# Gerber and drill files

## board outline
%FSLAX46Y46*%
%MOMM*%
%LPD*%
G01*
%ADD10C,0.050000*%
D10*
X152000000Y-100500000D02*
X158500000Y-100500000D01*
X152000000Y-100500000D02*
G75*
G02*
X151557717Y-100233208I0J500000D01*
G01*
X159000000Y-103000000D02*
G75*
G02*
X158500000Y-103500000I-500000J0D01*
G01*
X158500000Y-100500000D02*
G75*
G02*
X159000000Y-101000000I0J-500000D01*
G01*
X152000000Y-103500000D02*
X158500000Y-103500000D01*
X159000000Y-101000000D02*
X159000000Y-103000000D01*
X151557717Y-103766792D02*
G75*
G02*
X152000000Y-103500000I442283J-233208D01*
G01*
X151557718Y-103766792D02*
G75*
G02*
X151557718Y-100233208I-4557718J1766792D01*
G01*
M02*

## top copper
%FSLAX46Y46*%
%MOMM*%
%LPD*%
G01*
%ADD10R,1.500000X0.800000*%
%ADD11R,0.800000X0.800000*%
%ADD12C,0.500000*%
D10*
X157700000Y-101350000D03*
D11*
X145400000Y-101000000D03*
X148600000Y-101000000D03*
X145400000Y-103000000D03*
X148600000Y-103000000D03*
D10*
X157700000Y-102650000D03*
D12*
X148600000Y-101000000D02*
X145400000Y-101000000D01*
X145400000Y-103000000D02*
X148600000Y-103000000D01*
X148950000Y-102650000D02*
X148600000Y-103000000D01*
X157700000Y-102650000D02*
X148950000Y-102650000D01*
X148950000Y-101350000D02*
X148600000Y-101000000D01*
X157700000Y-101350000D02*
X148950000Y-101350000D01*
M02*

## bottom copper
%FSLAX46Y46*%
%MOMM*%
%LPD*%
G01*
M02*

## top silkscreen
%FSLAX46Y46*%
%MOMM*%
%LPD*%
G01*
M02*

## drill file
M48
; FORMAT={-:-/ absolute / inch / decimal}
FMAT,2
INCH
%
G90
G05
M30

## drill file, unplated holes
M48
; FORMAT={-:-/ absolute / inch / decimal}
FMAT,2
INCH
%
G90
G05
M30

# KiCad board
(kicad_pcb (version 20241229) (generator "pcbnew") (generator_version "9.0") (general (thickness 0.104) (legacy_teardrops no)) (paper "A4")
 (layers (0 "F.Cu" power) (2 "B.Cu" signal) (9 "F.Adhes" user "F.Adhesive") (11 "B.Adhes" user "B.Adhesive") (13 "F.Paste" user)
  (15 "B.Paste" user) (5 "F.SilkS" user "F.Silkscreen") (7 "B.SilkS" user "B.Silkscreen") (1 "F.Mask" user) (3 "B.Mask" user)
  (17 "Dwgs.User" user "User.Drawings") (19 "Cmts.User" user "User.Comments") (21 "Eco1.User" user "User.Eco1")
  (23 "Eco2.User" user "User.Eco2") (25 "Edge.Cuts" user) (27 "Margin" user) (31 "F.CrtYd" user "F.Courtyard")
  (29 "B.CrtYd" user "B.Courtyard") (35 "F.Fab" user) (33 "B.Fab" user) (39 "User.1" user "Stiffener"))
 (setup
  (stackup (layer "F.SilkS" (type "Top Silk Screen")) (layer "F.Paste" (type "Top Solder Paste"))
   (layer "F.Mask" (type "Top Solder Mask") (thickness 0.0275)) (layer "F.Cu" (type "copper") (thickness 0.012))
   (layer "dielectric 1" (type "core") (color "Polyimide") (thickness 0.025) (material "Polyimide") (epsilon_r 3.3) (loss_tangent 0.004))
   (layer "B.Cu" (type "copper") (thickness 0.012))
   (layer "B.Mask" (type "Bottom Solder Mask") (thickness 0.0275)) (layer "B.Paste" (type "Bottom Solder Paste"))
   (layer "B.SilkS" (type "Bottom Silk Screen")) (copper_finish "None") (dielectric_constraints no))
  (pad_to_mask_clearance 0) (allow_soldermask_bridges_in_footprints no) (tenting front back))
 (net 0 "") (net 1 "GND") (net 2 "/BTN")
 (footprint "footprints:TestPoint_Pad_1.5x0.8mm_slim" (layer "F.Cu") (at 157.7 101.35)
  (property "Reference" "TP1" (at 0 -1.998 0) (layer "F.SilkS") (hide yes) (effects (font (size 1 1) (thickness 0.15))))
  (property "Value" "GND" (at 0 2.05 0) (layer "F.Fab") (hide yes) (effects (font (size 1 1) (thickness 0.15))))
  (pad "1" smd rect (at 0 0) (size 1.5 0.8) (layers "F.Cu" "F.Mask") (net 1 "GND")))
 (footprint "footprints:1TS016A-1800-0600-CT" (layer "F.Cu") (at 147 102 90)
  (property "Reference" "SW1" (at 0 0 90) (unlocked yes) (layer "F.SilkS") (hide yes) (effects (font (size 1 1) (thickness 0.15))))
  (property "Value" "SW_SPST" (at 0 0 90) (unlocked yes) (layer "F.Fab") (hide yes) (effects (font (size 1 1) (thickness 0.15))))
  (pad "1" smd rect (at 1 -1.6 90) (size 0.8 0.8) (layers "F.Cu" "F.Mask" "F.Paste") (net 1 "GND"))
  (pad "1" smd rect (at 1 1.6 90) (size 0.8 0.8) (layers "F.Cu" "F.Mask" "F.Paste") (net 1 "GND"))
  (pad "2" smd rect (at -1 -1.6 90) (size 0.8 0.8) (layers "F.Cu" "F.Mask" "F.Paste") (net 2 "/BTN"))
  (pad "2" smd rect (at -1 1.6 90) (size 0.8 0.8) (layers "F.Cu" "F.Mask" "F.Paste") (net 2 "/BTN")))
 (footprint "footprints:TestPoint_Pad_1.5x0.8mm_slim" (layer "F.Cu") (at 157.7 102.65)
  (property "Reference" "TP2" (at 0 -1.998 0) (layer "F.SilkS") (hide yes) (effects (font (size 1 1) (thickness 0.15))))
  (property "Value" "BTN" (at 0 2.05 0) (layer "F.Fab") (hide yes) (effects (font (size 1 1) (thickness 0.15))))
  (pad "1" smd rect (at 0 0) (size 1.5 0.8) (layers "F.Cu" "F.Mask") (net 2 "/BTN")))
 (gr_line (start 152 100.5) (end 158.5 100.5) (stroke (width 0.05) (type default)) (layer "Edge.Cuts"))
 (gr_arc (start 152 100.5) (mid 151.74174 100.428138) (end 151.557717 100.233208) (stroke (width 0.05) (type default)) (layer "Edge.Cuts"))
 (gr_arc (start 159 103) (mid 158.853553 103.353553) (end 158.5 103.5) (stroke (width 0.05) (type default)) (layer "Edge.Cuts"))
 (gr_arc (start 158.5 100.5) (mid 158.853553 100.646447) (end 159 101) (stroke (width 0.05) (type default)) (layer "Edge.Cuts"))
 (gr_line (start 152 103.5) (end 158.5 103.5) (stroke (width 0.05) (type default)) (layer "Edge.Cuts"))
 (gr_line (start 159 101) (end 159 103) (stroke (width 0.05) (type default)) (layer "Edge.Cuts"))
 (gr_arc (start 151.557717 103.766792) (mid 151.74174 103.571862) (end 152 103.5) (stroke (width 0.05) (type default)) (layer "Edge.Cuts"))
 (gr_arc (start 151.557718 103.766792) (mid 142.111816 102) (end 151.557717 100.233208) (stroke (width 0.05) (type default))
  (layer "Edge.Cuts"))
 (segment (start 148.95 101.35) (end 148.6 101) (width 0.5) (layer "F.Cu") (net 1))
 (segment (start 157.7 101.35) (end 148.95 101.35) (width 0.5) (layer "F.Cu") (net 1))
 (segment (start 148.6 101) (end 145.4 101) (width 0.5) (layer "F.Cu") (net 1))
 (segment (start 148.95 102.65) (end 148.6 103) (width 0.5) (layer "F.Cu") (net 2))
 (segment (start 157.7 102.65) (end 148.95 102.65) (width 0.5) (layer "F.Cu") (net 2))
 (segment (start 145.4 103) (end 148.6 103) (width 0.5) (layer "F.Cu") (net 2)))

